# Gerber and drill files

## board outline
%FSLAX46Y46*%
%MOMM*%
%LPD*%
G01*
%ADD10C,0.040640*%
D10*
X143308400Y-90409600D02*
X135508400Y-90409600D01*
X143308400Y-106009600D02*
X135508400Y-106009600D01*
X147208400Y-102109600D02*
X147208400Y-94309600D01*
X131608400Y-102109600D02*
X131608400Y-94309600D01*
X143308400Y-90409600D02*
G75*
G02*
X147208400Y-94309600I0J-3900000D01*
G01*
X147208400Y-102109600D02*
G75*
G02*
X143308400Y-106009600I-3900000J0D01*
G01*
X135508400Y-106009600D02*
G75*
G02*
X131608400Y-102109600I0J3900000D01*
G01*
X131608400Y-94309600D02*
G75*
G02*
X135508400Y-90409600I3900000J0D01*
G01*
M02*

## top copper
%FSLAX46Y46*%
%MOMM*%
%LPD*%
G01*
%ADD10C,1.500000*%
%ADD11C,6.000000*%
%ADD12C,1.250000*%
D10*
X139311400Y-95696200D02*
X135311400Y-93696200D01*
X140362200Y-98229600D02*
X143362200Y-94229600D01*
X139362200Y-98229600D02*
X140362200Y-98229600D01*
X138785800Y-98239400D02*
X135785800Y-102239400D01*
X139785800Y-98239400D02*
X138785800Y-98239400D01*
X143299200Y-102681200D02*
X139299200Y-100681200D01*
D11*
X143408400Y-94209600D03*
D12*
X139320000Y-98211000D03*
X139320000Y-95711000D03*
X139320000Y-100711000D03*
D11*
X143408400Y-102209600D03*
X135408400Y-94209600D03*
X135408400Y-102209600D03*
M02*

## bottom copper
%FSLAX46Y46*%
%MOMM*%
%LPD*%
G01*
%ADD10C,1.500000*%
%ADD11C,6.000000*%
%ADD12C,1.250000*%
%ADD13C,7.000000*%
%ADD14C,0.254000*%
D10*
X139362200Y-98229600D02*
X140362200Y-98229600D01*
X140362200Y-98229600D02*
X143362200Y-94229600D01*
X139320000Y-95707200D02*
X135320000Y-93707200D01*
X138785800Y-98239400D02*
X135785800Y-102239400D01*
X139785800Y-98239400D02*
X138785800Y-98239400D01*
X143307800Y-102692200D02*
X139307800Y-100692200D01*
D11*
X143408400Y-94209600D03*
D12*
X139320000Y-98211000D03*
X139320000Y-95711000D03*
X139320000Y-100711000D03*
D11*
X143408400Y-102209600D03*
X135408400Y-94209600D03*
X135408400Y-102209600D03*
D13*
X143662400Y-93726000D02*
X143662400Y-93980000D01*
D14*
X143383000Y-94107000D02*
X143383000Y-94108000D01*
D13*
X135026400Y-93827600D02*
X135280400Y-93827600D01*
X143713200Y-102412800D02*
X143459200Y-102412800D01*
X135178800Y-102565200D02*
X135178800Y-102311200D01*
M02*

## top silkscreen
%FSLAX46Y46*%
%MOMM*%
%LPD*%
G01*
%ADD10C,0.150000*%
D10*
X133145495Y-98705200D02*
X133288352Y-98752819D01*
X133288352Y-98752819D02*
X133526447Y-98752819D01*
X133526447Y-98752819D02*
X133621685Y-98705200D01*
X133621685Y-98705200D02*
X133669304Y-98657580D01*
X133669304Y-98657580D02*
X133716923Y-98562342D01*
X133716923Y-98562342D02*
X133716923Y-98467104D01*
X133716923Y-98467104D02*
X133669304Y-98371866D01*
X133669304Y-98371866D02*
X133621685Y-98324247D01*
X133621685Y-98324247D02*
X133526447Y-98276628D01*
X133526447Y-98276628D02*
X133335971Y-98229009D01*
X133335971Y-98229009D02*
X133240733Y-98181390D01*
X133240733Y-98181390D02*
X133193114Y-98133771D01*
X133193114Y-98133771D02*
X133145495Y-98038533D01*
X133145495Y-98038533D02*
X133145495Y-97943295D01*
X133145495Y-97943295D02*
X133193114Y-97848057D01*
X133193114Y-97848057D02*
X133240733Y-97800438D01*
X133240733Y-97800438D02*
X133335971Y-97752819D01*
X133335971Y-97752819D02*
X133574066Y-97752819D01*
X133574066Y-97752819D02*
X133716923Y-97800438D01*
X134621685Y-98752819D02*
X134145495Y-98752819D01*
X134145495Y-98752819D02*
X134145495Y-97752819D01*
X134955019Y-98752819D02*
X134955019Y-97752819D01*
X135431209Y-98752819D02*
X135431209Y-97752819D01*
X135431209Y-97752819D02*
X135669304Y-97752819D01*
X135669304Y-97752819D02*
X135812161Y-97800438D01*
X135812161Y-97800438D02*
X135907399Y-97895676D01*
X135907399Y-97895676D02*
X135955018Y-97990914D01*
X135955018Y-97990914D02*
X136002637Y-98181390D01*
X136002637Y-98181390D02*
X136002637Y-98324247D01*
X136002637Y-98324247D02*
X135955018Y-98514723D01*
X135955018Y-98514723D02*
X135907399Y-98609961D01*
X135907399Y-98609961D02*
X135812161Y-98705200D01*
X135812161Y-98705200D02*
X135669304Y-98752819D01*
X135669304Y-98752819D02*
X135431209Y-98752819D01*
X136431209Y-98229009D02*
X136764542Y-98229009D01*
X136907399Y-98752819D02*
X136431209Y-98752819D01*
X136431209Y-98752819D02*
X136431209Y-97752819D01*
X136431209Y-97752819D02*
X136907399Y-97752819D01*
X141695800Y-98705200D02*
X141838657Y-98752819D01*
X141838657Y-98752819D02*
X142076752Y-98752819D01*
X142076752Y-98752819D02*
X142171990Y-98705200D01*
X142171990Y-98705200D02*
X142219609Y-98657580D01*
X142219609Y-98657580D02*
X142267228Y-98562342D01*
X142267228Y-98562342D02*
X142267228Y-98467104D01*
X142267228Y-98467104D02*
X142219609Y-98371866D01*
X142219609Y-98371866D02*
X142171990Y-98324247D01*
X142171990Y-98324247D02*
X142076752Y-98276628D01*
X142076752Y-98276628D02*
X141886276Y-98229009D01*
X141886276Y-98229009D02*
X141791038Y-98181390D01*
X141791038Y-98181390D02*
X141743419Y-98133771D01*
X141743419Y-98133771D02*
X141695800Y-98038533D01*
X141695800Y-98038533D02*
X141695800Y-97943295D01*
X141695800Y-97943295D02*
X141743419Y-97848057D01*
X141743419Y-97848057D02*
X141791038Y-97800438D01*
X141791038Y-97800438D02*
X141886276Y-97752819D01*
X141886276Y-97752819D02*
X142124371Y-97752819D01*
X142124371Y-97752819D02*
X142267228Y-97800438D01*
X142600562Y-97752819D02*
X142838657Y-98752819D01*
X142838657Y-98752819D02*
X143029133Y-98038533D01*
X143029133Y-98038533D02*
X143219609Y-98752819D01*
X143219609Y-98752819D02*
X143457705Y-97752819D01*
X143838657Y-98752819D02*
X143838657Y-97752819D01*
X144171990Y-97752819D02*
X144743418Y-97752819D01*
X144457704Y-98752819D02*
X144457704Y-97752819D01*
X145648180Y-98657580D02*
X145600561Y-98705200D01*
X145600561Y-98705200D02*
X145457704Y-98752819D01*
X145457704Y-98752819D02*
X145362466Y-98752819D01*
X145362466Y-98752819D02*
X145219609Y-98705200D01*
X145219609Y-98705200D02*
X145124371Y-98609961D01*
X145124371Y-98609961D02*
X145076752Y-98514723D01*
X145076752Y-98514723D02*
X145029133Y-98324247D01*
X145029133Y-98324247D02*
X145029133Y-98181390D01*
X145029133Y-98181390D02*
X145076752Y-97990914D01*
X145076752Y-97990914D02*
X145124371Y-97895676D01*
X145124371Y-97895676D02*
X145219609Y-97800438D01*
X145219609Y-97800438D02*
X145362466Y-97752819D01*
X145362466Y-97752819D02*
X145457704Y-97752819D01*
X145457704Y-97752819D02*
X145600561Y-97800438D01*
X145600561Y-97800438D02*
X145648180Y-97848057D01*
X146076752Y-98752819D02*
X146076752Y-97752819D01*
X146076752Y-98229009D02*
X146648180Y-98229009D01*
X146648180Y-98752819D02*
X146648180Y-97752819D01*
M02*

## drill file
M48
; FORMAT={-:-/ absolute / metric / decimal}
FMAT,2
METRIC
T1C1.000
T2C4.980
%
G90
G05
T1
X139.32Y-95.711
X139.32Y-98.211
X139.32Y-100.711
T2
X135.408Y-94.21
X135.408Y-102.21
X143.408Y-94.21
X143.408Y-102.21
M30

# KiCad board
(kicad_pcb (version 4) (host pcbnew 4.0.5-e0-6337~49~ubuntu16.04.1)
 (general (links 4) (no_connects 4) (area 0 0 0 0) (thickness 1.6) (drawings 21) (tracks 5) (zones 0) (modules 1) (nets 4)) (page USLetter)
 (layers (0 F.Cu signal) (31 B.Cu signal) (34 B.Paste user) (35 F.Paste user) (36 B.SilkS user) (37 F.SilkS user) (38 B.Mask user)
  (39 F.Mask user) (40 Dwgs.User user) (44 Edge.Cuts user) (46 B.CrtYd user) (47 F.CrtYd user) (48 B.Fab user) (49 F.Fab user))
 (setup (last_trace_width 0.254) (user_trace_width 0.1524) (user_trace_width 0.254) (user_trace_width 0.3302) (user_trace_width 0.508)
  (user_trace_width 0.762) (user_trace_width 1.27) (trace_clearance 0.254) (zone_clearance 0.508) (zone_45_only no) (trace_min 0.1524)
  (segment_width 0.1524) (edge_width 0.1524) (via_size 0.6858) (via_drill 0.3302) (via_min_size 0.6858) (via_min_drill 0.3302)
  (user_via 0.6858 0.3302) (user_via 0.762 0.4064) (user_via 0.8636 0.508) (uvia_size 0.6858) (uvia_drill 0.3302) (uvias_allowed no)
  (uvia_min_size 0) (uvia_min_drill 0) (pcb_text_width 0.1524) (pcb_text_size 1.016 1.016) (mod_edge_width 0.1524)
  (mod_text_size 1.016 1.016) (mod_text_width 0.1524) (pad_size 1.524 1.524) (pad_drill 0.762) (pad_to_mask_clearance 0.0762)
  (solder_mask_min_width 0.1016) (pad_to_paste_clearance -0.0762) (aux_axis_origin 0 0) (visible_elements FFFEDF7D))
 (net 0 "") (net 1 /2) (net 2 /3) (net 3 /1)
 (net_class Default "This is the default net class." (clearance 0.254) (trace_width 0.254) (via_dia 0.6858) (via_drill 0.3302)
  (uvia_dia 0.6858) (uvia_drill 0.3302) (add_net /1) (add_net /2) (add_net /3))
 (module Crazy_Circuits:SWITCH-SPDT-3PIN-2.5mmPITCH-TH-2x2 (layer F.Cu) (at 135.4084 102.2096)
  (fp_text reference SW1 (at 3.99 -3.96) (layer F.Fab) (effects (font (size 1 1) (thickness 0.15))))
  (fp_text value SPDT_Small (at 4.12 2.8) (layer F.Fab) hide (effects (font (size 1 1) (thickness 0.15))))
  (fp_line (start 3.903 -6.5134) (end -0.097 -8.5134) (layer F.Cu) (width 1.5))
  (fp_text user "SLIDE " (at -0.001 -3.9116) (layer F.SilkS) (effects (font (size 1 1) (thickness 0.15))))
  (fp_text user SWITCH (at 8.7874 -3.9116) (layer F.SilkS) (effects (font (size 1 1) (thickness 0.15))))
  (fp_line (start 3.9538 -3.98) (end 4.9538 -3.98) (layer B.Cu) (width 1.5))
  (fp_line (start 4.9538 -3.98) (end 7.9538 -7.98) (layer B.Cu) (width 1.5))
  (fp_line (start 7.9 -11.8) (end 0.1 -11.8) (layer Edge.Cuts) (width 0.04064))
  (fp_line (start 7.9 3.8) (end 0.1 3.8) (layer Edge.Cuts) (width 0.04064))
  (fp_line (start 11.8 -0.1) (end 11.8 -7.9) (layer Edge.Cuts) (width 0.04064))
  (fp_line (start -3.8 -0.1) (end -3.8 -7.9) (layer Edge.Cuts) (width 0.04064))
  (fp_arc (start 7.9 -7.9) (end 7.9 -11.8) (angle 90) (layer Edge.Cuts) (width 0.04064))
  (fp_arc (start 7.9 -0.1) (end 11.8 -0.1) (angle 90) (layer Edge.Cuts) (width 0.04064))
  (fp_arc (start 0.1 -0.1) (end 0.1 3.8) (angle 90) (layer Edge.Cuts) (width 0.04064))
  (fp_arc (start 0.1 -7.9) (end -3.8 -7.9) (angle 90) (layer Edge.Cuts) (width 0.04064))
  (fp_line (start 4.9538 -3.98) (end 7.9538 -7.98) (layer F.Cu) (width 1.5))
  (fp_line (start 3.9538 -3.98) (end 4.9538 -3.98) (layer F.Cu) (width 1.5))
  (fp_line (start 3.9116 -6.5024) (end -0.0884 -8.5024) (layer B.Cu) (width 1.5))
  (fp_line (start 3.3774 -3.9702) (end 0.3774 0.0298) (layer F.Cu) (width 1.5))
  (fp_line (start 3.3774 -3.9702) (end 0.3774 0.0298) (layer B.Cu) (width 1.5))
  (fp_line (start 4.3774 -3.9702) (end 3.3774 -3.9702) (layer B.Cu) (width 1.5))
  (fp_line (start 4.3774 -3.9702) (end 3.3774 -3.9702) (layer F.Cu) (width 1.5))
  (fp_line (start 7.8908 0.4716) (end 3.8908 -1.5284) (layer F.Cu) (width 1.5))
  (fp_line (start 7.8994 0.4826) (end 3.8994 -1.5174) (layer B.Cu) (width 1.5))
  (pad 2 thru_hole circle (at 8 -8) (size 6 6) (drill 4.98) (layers *.Cu *.Mask) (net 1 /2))
  (pad 2 thru_hole circle (at 3.9116 -3.9986 270) (size 1.25 1.25) (drill 1) (layers *.Cu *.Mask) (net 1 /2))
  (pad 3 thru_hole circle (at 3.9116 -6.4986 270) (size 1.25 1.25) (drill 1) (layers *.Cu *.Mask) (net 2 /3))
  (pad 1 thru_hole circle (at 3.9116 -1.4986 270) (size 1.25 1.25) (drill 1) (layers *.Cu *.Mask) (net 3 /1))
  (pad 1 thru_hole circle (at 8 0) (size 6 6) (drill 4.98) (layers *.Cu *.Mask) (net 3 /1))
  (pad 3 thru_hole circle (at 0 -8) (size 6 6) (drill 4.98) (layers *.Cu *.Mask) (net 2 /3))
  (pad 2 thru_hole circle (at 0 0) (size 6 6) (drill 4.98) (layers *.Cu *.Mask) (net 1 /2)))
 (segment (start 143.6624 93.726) (end 143.6624 93.98) (width 7) (layer B.Cu) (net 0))
 (segment (start 143.383 94.107) (end 143.383 94.108) (width 0.254) (layer B.Cu) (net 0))
 (segment (start 135.0264 93.8276) (end 135.2804 93.8276) (width 7) (layer B.Cu) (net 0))
 (segment (start 143.7132 102.4128) (end 143.4592 102.4128) (width 7) (layer B.Cu) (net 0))
 (segment (start 135.1788 102.5652) (end 135.1788 102.3112) (width 7) (layer B.Cu) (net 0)))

